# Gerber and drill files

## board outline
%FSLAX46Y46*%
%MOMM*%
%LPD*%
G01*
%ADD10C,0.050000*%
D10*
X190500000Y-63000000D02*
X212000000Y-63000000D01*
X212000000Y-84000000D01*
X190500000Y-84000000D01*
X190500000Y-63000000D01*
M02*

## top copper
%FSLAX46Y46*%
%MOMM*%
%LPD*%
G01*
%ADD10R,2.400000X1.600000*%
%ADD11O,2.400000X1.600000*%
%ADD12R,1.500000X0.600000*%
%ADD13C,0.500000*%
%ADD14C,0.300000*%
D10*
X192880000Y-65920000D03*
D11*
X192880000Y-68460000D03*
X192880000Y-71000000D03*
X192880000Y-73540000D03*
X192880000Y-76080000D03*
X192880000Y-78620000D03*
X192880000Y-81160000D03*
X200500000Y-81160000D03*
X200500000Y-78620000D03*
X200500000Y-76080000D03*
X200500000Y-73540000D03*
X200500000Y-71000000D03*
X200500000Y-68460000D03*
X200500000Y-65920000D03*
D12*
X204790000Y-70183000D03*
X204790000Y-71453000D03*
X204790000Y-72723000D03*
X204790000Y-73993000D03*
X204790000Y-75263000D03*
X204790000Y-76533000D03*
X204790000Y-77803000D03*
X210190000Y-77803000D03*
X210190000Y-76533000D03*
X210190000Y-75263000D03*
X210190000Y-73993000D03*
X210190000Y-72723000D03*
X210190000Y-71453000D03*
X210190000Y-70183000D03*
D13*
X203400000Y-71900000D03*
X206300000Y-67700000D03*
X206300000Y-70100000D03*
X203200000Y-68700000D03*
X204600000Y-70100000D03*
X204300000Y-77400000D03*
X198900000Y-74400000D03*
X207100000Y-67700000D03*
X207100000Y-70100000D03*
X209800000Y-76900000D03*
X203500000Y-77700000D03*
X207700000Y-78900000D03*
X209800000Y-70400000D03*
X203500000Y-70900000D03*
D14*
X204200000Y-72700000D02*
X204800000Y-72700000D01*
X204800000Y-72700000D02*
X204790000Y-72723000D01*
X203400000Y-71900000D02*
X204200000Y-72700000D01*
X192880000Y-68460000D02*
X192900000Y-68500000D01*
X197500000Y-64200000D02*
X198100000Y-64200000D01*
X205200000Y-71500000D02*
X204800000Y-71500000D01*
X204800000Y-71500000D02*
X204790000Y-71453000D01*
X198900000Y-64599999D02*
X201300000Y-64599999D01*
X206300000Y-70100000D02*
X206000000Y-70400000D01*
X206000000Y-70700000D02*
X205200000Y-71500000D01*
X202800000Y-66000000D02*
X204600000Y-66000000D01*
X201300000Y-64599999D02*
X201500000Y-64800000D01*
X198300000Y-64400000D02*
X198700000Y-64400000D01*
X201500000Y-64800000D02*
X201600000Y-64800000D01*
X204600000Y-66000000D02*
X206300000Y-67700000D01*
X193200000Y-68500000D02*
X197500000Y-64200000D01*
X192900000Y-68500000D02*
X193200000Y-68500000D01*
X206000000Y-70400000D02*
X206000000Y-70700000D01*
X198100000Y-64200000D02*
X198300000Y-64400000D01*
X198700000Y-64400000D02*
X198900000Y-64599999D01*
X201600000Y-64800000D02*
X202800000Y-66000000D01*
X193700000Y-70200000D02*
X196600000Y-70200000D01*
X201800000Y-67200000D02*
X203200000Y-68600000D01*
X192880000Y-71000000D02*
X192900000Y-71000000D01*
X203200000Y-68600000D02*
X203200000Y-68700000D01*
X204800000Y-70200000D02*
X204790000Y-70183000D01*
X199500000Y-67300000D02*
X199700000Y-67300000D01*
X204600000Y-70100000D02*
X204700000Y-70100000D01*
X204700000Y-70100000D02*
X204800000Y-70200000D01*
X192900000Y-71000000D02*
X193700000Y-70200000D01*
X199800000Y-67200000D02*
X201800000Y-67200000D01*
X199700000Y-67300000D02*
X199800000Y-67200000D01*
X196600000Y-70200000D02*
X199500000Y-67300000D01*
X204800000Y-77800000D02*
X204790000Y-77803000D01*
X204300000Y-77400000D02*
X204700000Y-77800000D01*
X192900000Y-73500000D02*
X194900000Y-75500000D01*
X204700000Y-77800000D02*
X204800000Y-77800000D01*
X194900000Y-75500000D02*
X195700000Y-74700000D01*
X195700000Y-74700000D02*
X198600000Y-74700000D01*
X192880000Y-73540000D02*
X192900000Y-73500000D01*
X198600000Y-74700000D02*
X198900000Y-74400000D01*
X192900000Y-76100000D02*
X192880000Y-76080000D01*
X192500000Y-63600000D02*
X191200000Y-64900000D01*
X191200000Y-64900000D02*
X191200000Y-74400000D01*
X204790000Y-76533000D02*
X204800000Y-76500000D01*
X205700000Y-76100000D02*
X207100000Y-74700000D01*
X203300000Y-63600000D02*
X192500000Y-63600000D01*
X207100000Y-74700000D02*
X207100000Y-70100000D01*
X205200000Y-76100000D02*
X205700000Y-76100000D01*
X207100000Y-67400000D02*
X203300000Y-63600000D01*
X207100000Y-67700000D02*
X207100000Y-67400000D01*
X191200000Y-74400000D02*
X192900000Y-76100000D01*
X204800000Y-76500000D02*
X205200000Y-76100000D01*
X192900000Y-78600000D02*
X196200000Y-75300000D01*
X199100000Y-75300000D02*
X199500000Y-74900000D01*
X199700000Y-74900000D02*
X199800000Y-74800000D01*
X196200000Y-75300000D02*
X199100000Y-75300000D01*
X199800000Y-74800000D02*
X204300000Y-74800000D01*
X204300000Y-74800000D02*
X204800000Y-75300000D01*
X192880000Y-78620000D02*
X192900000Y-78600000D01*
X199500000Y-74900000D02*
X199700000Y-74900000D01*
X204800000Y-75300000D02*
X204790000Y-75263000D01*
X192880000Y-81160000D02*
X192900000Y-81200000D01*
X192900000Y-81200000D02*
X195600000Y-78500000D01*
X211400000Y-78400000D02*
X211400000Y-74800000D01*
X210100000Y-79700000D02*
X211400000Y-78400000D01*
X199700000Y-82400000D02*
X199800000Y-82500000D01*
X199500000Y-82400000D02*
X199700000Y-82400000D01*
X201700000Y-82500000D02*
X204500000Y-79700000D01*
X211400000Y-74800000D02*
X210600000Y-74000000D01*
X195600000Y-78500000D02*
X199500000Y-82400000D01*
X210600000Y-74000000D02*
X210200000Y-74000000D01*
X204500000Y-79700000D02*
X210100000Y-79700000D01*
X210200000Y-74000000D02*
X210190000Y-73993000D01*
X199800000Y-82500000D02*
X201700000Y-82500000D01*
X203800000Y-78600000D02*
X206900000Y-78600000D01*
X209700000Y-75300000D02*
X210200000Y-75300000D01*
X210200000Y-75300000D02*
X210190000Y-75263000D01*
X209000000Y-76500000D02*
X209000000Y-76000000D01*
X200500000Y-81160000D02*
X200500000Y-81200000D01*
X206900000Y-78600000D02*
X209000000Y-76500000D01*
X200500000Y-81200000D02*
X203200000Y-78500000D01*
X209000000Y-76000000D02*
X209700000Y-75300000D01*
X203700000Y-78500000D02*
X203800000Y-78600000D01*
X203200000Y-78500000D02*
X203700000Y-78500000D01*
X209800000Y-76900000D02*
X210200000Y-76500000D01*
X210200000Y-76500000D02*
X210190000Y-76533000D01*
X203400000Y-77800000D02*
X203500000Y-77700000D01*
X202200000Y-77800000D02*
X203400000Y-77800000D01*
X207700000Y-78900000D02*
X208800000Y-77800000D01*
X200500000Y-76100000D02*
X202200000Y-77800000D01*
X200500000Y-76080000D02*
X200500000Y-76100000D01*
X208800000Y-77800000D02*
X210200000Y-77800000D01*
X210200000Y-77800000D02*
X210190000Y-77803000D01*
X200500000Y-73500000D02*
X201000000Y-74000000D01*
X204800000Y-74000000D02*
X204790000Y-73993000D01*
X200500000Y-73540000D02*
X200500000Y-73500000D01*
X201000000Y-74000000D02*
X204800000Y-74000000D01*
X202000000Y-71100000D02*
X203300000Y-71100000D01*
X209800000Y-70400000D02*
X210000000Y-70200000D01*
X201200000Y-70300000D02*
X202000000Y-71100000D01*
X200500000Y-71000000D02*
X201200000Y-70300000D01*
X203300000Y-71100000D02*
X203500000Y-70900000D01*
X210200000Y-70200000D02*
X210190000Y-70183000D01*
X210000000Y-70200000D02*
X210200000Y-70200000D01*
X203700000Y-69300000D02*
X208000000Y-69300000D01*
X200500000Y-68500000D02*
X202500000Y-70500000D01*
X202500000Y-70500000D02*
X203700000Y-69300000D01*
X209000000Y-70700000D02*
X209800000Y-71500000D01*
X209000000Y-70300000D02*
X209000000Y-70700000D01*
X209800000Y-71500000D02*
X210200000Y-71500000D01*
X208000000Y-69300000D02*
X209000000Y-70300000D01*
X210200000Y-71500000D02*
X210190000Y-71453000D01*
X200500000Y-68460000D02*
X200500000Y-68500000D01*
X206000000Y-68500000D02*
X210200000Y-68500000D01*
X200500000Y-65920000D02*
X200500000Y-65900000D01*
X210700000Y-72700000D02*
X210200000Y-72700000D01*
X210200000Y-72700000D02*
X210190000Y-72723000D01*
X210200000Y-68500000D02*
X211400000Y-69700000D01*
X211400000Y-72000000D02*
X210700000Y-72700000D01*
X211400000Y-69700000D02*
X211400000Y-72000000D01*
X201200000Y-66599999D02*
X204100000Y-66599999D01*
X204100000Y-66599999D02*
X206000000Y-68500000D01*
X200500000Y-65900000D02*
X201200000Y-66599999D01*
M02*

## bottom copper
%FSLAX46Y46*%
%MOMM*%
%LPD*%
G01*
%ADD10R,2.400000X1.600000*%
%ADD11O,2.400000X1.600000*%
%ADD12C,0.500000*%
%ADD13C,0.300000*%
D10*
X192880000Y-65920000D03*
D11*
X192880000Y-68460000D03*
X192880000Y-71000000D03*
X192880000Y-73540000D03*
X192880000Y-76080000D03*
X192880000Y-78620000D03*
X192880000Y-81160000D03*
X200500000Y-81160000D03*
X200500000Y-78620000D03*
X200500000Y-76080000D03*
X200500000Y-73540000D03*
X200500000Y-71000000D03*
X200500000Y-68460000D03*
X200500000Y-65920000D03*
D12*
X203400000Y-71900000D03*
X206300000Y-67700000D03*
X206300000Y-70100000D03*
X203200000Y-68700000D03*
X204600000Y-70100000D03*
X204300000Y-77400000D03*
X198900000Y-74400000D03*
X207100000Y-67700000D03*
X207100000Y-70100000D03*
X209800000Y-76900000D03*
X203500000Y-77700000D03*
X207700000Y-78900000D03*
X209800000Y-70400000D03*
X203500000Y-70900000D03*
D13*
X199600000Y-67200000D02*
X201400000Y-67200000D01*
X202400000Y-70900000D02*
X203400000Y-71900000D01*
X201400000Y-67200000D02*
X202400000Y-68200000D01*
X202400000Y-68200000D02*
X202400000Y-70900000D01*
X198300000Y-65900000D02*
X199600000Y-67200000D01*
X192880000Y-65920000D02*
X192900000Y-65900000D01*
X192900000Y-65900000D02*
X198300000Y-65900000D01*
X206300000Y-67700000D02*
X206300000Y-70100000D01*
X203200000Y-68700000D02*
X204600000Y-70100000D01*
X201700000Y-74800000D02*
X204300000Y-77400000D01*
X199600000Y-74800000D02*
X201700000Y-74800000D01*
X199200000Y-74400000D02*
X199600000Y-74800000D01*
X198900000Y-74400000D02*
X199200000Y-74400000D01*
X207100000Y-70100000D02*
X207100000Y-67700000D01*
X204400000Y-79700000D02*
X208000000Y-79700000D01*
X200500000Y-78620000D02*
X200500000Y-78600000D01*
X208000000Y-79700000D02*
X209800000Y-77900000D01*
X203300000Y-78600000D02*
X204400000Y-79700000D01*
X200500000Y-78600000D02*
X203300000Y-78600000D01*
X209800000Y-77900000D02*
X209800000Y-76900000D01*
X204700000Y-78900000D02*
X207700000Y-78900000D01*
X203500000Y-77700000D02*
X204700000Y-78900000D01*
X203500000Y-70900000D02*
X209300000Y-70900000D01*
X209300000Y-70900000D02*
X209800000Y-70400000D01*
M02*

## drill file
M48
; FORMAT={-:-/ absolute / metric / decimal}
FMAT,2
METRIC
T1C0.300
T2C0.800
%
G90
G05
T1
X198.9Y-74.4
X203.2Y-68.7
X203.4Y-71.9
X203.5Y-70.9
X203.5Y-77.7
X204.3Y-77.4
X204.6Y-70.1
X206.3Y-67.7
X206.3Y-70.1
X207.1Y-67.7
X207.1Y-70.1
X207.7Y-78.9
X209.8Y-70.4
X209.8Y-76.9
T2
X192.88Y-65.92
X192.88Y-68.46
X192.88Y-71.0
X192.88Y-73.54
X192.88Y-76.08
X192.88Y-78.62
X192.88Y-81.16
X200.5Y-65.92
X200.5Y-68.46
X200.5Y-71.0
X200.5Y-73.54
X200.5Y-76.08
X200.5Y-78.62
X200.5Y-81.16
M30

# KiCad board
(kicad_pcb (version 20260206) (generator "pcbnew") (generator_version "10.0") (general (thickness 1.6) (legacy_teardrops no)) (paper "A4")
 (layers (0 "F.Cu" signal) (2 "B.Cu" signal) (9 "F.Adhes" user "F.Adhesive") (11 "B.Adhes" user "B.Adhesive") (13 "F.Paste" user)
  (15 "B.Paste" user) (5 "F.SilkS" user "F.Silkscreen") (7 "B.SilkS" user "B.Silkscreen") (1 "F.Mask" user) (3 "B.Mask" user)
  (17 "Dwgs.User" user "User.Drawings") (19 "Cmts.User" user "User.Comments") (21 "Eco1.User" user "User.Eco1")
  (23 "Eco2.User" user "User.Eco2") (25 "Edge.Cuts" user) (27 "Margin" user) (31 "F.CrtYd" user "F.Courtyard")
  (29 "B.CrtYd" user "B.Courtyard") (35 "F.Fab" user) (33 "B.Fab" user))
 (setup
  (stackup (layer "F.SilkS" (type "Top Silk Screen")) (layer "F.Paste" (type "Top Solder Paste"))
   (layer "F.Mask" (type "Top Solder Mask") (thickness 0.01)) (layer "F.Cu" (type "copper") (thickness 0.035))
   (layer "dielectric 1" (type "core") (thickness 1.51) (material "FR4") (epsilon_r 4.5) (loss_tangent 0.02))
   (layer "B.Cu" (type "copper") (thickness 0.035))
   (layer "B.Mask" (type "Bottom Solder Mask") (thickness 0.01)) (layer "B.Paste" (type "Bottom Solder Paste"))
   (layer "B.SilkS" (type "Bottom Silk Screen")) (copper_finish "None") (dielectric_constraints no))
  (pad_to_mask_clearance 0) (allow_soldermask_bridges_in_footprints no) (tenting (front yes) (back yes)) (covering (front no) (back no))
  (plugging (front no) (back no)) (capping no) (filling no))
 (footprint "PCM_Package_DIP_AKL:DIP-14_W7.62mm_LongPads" (layer "F.Cu") (at 192.88 65.92)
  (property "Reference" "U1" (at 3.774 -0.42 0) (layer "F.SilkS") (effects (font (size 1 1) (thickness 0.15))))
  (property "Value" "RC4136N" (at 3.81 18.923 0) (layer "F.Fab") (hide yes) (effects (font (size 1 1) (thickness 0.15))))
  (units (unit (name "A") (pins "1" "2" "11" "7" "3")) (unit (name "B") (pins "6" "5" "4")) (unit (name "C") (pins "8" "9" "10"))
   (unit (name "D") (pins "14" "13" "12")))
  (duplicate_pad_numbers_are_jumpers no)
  (pad "1" thru_hole rect (at 0 0) (size 2.4 1.6) (drill 0.8) (layers "*.Cu" "*.Mask") (remove_unused_layers no) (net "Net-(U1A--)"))
  (pad "2" thru_hole oval (at 0 2.54) (size 2.4 1.6) (drill 0.8) (layers "*.Cu" "*.Mask") (remove_unused_layers no) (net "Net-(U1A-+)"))
  (pad "3" thru_hole oval (at 0 5.08) (size 2.4 1.6) (drill 0.8) (layers "*.Cu" "*.Mask") (remove_unused_layers no) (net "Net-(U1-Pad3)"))
  (pad "4" thru_hole oval (at 0 7.62) (size 2.4 1.6) (drill 0.8) (layers "*.Cu" "*.Mask") (remove_unused_layers no) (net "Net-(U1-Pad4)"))
  (pad "5" thru_hole oval (at 0 10.16) (size 2.4 1.6) (drill 0.8) (layers "*.Cu" "*.Mask") (remove_unused_layers no) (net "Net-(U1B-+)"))
  (pad "6" thru_hole oval (at 0 12.7) (size 2.4 1.6) (drill 0.8) (layers "*.Cu" "*.Mask") (remove_unused_layers no) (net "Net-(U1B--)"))
  (pad "7" thru_hole oval (at 0 15.24) (size 2.4 1.6) (drill 0.8) (layers "*.Cu" "*.Mask") (remove_unused_layers no) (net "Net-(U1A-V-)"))
  (pad "8" thru_hole oval (at 7.62 15.24) (size 2.4 1.6) (drill 0.8) (layers "*.Cu" "*.Mask") (remove_unused_layers no) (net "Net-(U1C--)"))
  (pad "9" thru_hole oval (at 7.62 12.7) (size 2.4 1.6) (drill 0.8) (layers "*.Cu" "*.Mask") (remove_unused_layers no) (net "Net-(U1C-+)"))
  (pad "10" thru_hole oval (at 7.62 10.16) (size 2.4 1.6) (drill 0.8) (layers "*.Cu" "*.Mask") (remove_unused_layers no)
   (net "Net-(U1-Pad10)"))
  (pad "11" thru_hole oval (at 7.62 7.62) (size 2.4 1.6) (drill 0.8) (layers "*.Cu" "*.Mask") (remove_unused_layers no) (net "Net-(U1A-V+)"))
  (pad "12" thru_hole oval (at 7.62 5.08) (size 2.4 1.6) (drill 0.8) (layers "*.Cu" "*.Mask") (remove_unused_layers no)
   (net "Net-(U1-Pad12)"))
  (pad "13" thru_hole oval (at 7.62 2.54) (size 2.4 1.6) (drill 0.8) (layers "*.Cu" "*.Mask") (remove_unused_layers no) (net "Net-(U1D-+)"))
  (pad "14" thru_hole oval (at 7.62 0) (size 2.4 1.6) (drill 0.8) (layers "*.Cu" "*.Mask") (remove_unused_layers no) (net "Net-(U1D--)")))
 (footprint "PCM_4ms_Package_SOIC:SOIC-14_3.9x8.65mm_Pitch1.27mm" (layer "F.Cu") (at 207.5 74)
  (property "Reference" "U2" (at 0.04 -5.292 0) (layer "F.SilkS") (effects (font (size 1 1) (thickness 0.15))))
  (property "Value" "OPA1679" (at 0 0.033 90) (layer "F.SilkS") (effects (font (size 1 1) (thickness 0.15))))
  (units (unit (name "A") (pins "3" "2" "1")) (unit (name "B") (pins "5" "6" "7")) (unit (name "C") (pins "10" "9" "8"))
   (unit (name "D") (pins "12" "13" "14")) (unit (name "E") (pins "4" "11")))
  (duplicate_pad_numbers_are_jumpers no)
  (pad "1" smd rect (at -2.71 -3.817) (size 1.5 0.6) (layers "F.Cu" "F.Mask" "F.Paste") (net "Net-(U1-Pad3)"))
  (pad "2" smd rect (at -2.71 -2.547) (size 1.5 0.6) (layers "F.Cu" "F.Mask" "F.Paste") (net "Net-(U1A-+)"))
  (pad "3" smd rect (at -2.71 -1.277) (size 1.5 0.6) (layers "F.Cu" "F.Mask" "F.Paste") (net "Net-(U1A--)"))
  (pad "4" smd rect (at -2.71 -0.007) (size 1.5 0.6) (layers "F.Cu" "F.Mask" "F.Paste") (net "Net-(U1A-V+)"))
  (pad "5" smd rect (at -2.71 1.263) (size 1.5 0.6) (layers "F.Cu" "F.Mask" "F.Paste") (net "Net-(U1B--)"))
  (pad "6" smd rect (at -2.71 2.533) (size 1.5 0.6) (layers "F.Cu" "F.Mask" "F.Paste") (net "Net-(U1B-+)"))
  (pad "7" smd rect (at -2.71 3.803) (size 1.5 0.6) (layers "F.Cu" "F.Mask" "F.Paste") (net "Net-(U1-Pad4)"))
  (pad "8" smd rect (at 2.69 3.803) (size 1.5 0.6) (layers "F.Cu" "F.Mask" "F.Paste") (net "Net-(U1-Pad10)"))
  (pad "9" smd rect (at 2.69 2.533) (size 1.5 0.6) (layers "F.Cu" "F.Mask" "F.Paste") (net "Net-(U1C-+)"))
  (pad "10" smd rect (at 2.69 1.263) (size 1.5 0.6) (layers "F.Cu" "F.Mask" "F.Paste") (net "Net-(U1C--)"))
  (pad "11" smd rect (at 2.69 -0.007) (size 1.5 0.6) (layers "F.Cu" "F.Mask" "F.Paste") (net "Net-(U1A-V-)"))
  (pad "12" smd rect (at 2.69 -1.277) (size 1.5 0.6) (layers "F.Cu" "F.Mask" "F.Paste") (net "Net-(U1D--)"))
  (pad "13" smd rect (at 2.69 -2.547) (size 1.5 0.6) (layers "F.Cu" "F.Mask" "F.Paste") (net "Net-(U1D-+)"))
  (pad "14" smd rect (at 2.69 -3.817) (size 1.5 0.6) (layers "F.Cu" "F.Mask" "F.Paste") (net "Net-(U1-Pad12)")))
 (gr_rect (start 190.5 63) (end 212 84) (stroke (width 0.05) (type default)) (fill no) (layer "Edge.Cuts"))
 (segment (start 204.2 72.7) (end 204.8 72.7) (width 0.3) (layer "F.Cu") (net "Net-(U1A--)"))
 (segment (start 204.8 72.7) (end 204.79 72.723) (width 0.3) (layer "F.Cu") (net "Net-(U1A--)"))
 (segment (start 203.4 71.9) (end 204.2 72.7) (width 0.3) (layer "F.Cu") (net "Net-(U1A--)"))
 (via (at 203.4 71.9) (size 0.5) (drill 0.3) (layers "F.Cu" "B.Cu") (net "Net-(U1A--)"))
 (segment (start 199.6 67.2) (end 201.4 67.2) (width 0.3) (layer "B.Cu") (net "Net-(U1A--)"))
 (segment (start 202.4 70.9) (end 203.4 71.9) (width 0.3) (layer "B.Cu") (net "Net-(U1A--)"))
 (segment (start 201.4 67.2) (end 202.4 68.2) (width 0.3) (layer "B.Cu") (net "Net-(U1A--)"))
 (segment (start 202.4 68.2) (end 202.4 70.9) (width 0.3) (layer "B.Cu") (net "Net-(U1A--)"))
 (segment (start 198.3 65.9) (end 199.6 67.2) (width 0.3) (layer "B.Cu") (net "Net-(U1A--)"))
 (segment (start 192.88 65.92) (end 192.9 65.9) (width 0.3) (layer "B.Cu") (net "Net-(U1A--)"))
 (segment (start 192.9 65.9) (end 198.3 65.9) (width 0.3) (layer "B.Cu") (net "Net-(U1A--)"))
 (segment (start 192.88 68.46) (end 192.9 68.5) (width 0.3) (layer "F.Cu") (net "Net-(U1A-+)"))
 (segment (start 197.5 64.2) (end 198.1 64.2) (width 0.3) (layer "F.Cu") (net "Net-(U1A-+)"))
 (segment (start 205.2 71.5) (end 204.8 71.5) (width 0.3) (layer "F.Cu") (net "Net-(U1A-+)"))
 (segment (start 204.8 71.5) (end 204.79 71.453) (width 0.3) (layer "F.Cu") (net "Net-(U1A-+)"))
 (segment (start 198.9 64.599999) (end 201.3 64.599999) (width 0.3) (layer "F.Cu") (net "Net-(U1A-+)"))
 (segment (start 206.3 70.1) (end 206 70.4) (width 0.3) (layer "F.Cu") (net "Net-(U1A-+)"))
 (segment (start 206 70.7) (end 205.2 71.5) (width 0.3) (layer "F.Cu") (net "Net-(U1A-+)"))
 (segment (start 202.8 66) (end 204.6 66) (width 0.3) (layer "F.Cu") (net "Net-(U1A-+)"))
 (segment (start 201.3 64.599999) (end 201.5 64.8) (width 0.3) (layer "F.Cu") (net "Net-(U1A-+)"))
 (segment (start 198.3 64.4) (end 198.7 64.4) (width 0.3) (layer "F.Cu") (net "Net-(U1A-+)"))
 (segment (start 201.5 64.8) (end 201.6 64.8) (width 0.3) (layer "F.Cu") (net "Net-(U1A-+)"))
 (segment (start 204.6 66) (end 206.3 67.7) (width 0.3) (layer "F.Cu") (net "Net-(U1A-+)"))
 (segment (start 193.2 68.5) (end 197.5 64.2) (width 0.3) (layer "F.Cu") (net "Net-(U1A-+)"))
 (segment (start 192.9 68.5) (end 193.2 68.5) (width 0.3) (layer "F.Cu") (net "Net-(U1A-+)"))
 (segment (start 206 70.4) (end 206 70.7) (width 0.3) (layer "F.Cu") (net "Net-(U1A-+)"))
 (segment (start 198.1 64.2) (end 198.3 64.4) (width 0.3) (layer "F.Cu") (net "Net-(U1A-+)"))
 (segment (start 198.7 64.4) (end 198.9 64.599999) (width 0.3) (layer "F.Cu") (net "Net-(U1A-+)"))
 (segment (start 201.6 64.8) (end 202.8 66) (width 0.3) (layer "F.Cu") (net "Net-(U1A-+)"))
 (via (at 206.3 67.7) (size 0.5) (drill 0.3) (layers "F.Cu" "B.Cu") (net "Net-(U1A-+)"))
 (via (at 206.3 70.1) (size 0.5) (drill 0.3) (layers "F.Cu" "B.Cu") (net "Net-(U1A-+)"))
 (segment (start 206.3 67.7) (end 206.3 70.1) (width 0.3) (layer "B.Cu") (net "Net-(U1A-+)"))
 (segment (start 193.7 70.2) (end 196.6 70.2) (width 0.3) (layer "F.Cu") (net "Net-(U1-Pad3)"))
 (segment (start 201.8 67.2) (end 203.2 68.6) (width 0.3) (layer "F.Cu") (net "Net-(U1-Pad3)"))
 (segment (start 192.88 71) (end 192.9 71) (width 0.3) (layer "F.Cu") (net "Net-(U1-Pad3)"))
 (segment (start 203.2 68.6) (end 203.2 68.7) (width 0.3) (layer "F.Cu") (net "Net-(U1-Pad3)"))
 (segment (start 204.8 70.2) (end 204.79 70.183) (width 0.3) (layer "F.Cu") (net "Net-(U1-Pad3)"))
 (segment (start 199.5 67.3) (end 199.7 67.3) (width 0.3) (layer "F.Cu") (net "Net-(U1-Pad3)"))
 (segment (start 204.6 70.1) (end 204.7 70.1) (width 0.3) (layer "F.Cu") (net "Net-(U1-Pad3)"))
 (segment (start 204.7 70.1) (end 204.8 70.2) (width 0.3) (layer "F.Cu") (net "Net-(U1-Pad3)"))
 (segment (start 192.9 71) (end 193.7 70.2) (width 0.3) (layer "F.Cu") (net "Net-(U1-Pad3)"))
 (segment (start 199.8 67.2) (end 201.8 67.2) (width 0.3) (layer "F.Cu") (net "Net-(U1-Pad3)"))
 (segment (start 199.7 67.3) (end 199.8 67.2) (width 0.3) (layer "F.Cu") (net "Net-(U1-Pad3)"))
 (segment (start 196.6 70.2) (end 199.5 67.3) (width 0.3) (layer "F.Cu") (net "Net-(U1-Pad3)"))
 (via (at 203.2 68.7) (size 0.5) (drill 0.3) (layers "F.Cu" "B.Cu") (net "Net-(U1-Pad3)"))
 (via (at 204.6 70.1) (size 0.5) (drill 0.3) (layers "F.Cu" "B.Cu") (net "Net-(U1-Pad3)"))
 (segment (start 203.2 68.7) (end 204.6 70.1) (width 0.3) (layer "B.Cu") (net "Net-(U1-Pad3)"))
 (segment (start 204.8 77.8) (end 204.79 77.803) (width 0.3) (layer "F.Cu") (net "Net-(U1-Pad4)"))
 (segment (start 204.3 77.4) (end 204.7 77.8) (width 0.3) (layer "F.Cu") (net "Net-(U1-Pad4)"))
 (segment (start 192.9 73.5) (end 194.9 75.5) (width 0.3) (layer "F.Cu") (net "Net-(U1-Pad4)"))
 (segment (start 204.7 77.8) (end 204.8 77.8) (width 0.3) (layer "F.Cu") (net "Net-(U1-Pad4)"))
 (segment (start 194.9 75.5) (end 195.7 74.7) (width 0.3) (layer "F.Cu") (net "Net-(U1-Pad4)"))
 (segment (start 195.7 74.7) (end 198.6 74.7) (width 0.3) (layer "F.Cu") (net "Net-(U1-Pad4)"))
 (segment (start 192.88 73.54) (end 192.9 73.5) (width 0.3) (layer "F.Cu") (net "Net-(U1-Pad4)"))
 (segment (start 198.6 74.7) (end 198.9 74.4) (width 0.3) (layer "F.Cu") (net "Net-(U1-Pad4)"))
 (via (at 204.3 77.4) (size 0.5) (drill 0.3) (layers "F.Cu" "B.Cu") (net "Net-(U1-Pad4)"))
 (via (at 198.9 74.4) (size 0.5) (drill 0.3) (layers "F.Cu" "B.Cu") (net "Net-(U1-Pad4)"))
 (segment (start 201.7 74.8) (end 204.3 77.4) (width 0.3) (layer "B.Cu") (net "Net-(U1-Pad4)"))
 (segment (start 199.6 74.8) (end 201.7 74.8) (width 0.3) (layer "B.Cu") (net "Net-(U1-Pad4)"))
 (segment (start 199.2 74.4) (end 199.6 74.8) (width 0.3) (layer "B.Cu") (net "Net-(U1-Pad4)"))
 (segment (start 198.9 74.4) (end 199.2 74.4) (width 0.3) (layer "B.Cu") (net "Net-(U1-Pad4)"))
 (segment (start 192.9 76.1) (end 192.88 76.08) (width 0.3) (layer "F.Cu") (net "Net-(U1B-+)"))
 (segment (start 192.5 63.6) (end 191.2 64.9) (width 0.3) (layer "F.Cu") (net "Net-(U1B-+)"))
 (segment (start 191.2 64.9) (end 191.2 74.4) (width 0.3) (layer "F.Cu") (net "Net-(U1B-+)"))
 (segment (start 204.79 76.533) (end 204.8 76.5) (width 0.3) (layer "F.Cu") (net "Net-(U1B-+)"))
 (segment (start 205.7 76.1) (end 207.1 74.7) (width 0.3) (layer "F.Cu") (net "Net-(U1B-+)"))
 (segment (start 203.3 63.6) (end 192.5 63.6) (width 0.3) (layer "F.Cu") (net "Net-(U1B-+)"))
 (segment (start 207.1 74.7) (end 207.1 70.1) (width 0.3) (layer "F.Cu") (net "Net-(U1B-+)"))
 (segment (start 205.2 76.1) (end 205.7 76.1) (width 0.3) (layer "F.Cu") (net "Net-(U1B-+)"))
 (segment (start 207.1 67.4) (end 203.3 63.6) (width 0.3) (layer "F.Cu") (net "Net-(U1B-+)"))
 (segment (start 207.1 67.7) (end 207.1 67.4) (width 0.3) (layer "F.Cu") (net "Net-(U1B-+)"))
 (segment (start 191.2 74.4) (end 192.9 76.1) (width 0.3) (layer "F.Cu") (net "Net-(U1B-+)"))
 (segment (start 204.8 76.5) (end 205.2 76.1) (width 0.3) (layer "F.Cu") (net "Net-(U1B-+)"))
 (via (at 207.1 67.7) (size 0.5) (drill 0.3) (layers "F.Cu" "B.Cu") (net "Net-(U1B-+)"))
 (via (at 207.1 70.1) (size 0.5) (drill 0.3) (layers "F.Cu" "B.Cu") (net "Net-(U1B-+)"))
 (segment (start 207.1 70.1) (end 207.1 67.7) (width 0.3) (layer "B.Cu") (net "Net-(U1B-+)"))
 (segment (start 192.9 78.6) (end 196.2 75.3) (width 0.3) (layer "F.Cu") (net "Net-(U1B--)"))
 (segment (start 199.1 75.3) (end 199.5 74.9) (width 0.3) (layer "F.Cu") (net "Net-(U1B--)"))
 (segment (start 199.7 74.9) (end 199.8 74.8) (width 0.3) (layer "F.Cu") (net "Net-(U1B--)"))
 (segment (start 196.2 75.3) (end 199.1 75.3) (width 0.3) (layer "F.Cu") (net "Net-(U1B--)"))
 (segment (start 199.8 74.8) (end 204.3 74.8) (width 0.3) (layer "F.Cu") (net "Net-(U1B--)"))
 (segment (start 204.3 74.8) (end 204.8 75.3) (width 0.3) (layer "F.Cu") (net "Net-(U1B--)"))
 (segment (start 192.88 78.62) (end 192.9 78.6) (width 0.3) (layer "F.Cu") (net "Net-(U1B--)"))
 (segment (start 199.5 74.9) (end 199.7 74.9) (width 0.3) (layer "F.Cu") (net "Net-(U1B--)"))
 (segment (start 204.8 75.3) (end 204.79 75.263) (width 0.3) (layer "F.Cu") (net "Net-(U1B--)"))
 (segment (start 192.88 81.16) (end 192.9 81.2) (width 0.3) (layer "F.Cu") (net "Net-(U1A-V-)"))
 (segment (start 192.9 81.2) (end 195.6 78.5) (width 0.3) (layer "F.Cu") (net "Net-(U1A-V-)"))
 (segment (start 211.4 78.4) (end 211.4 74.8) (width 0.3) (layer "F.Cu") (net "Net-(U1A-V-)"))
 (segment (start 210.1 79.7) (end 211.4 78.4) (width 0.3) (layer "F.Cu") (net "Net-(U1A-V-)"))
 (segment (start 199.7 82.4) (end 199.8 82.5) (width 0.3) (layer "F.Cu") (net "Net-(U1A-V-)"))
 (segment (start 199.5 82.4) (end 199.7 82.4) (width 0.3) (layer "F.Cu") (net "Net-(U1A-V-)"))
 (segment (start 201.7 82.5) (end 204.5 79.7) (width 0.3) (layer "F.Cu") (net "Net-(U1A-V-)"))
 (segment (start 211.4 74.8) (end 210.6 74) (width 0.3) (layer "F.Cu") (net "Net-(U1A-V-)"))
 (segment (start 195.6 78.5) (end 199.5 82.4) (width 0.3) (layer "F.Cu") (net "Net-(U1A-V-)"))
 (segment (start 210.6 74) (end 210.2 74) (width 0.3) (layer "F.Cu") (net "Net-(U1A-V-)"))
 (segment (start 204.5 79.7) (end 210.1 79.7) (width 0.3) (layer "F.Cu") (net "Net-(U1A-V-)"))
 (segment (start 210.2 74) (end 210.19 73.993) (width 0.3) (layer "F.Cu") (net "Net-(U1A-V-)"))
 (segment (start 199.8 82.5) (end 201.7 82.5) (width 0.3) (layer "F.Cu") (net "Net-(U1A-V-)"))
 (segment (start 203.8 78.6) (end 206.9 78.6) (width 0.3) (layer "F.Cu") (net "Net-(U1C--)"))
 (segment (start 209.7 75.3) (end 210.2 75.3) (width 0.3) (layer "F.Cu") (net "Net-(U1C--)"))
 (segment (start 210.2 75.3) (end 210.19 75.263) (width 0.3) (layer "F.Cu") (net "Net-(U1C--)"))
 (segment (start 209 76.5) (end 209 76) (width 0.3) (layer "F.Cu") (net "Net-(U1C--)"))
 (segment (start 200.5 81.16) (end 200.5 81.2) (width 0.3) (layer "F.Cu") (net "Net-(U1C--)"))
 (segment (start 206.9 78.6) (end 209 76.5) (width 0.3) (layer "F.Cu") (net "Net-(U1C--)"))
 (segment (start 200.5 81.2) (end 203.2 78.5) (width 0.3) (layer "F.Cu") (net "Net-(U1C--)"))
 (segment (start 209 76) (end 209.7 75.3) (width 0.3) (layer "F.Cu") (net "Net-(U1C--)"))
 (segment (start 203.7 78.5) (end 203.8 78.6) (width 0.3) (layer "F.Cu") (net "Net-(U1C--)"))
 (segment (start 203.2 78.5) (end 203.7 78.5) (width 0.3) (layer "F.Cu") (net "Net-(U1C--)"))
 (segment (start 209.8 76.9) (end 210.2 76.5) (width 0.3) (layer "F.Cu") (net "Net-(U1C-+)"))
 (segment (start 210.2 76.5) (end 210.19 76.533) (width 0.3) (layer "F.Cu") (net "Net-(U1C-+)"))
 (via (at 209.8 76.9) (size 0.5) (drill 0.3) (layers "F.Cu" "B.Cu") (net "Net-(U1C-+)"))
 (segment (start 204.4 79.7) (end 208 79.7) (width 0.3) (layer "B.Cu") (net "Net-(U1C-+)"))
 (segment (start 200.5 78.62) (end 200.5 78.6) (width 0.3) (layer "B.Cu") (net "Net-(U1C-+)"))
 (segment (start 208 79.7) (end 209.8 77.9) (width 0.3) (layer "B.Cu") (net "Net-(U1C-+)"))
 (segment (start 203.3 78.6) (end 204.4 79.7) (width 0.3) (layer "B.Cu") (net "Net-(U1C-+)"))
 (segment (start 200.5 78.6) (end 203.3 78.6) (width 0.3) (layer "B.Cu") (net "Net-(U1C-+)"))
 (segment (start 209.8 77.9) (end 209.8 76.9) (width 0.3) (layer "B.Cu") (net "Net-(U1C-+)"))
 (segment (start 203.4 77.8) (end 203.5 77.7) (width 0.3) (layer "F.Cu") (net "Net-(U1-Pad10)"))
 (segment (start 202.2 77.8) (end 203.4 77.8) (width 0.3) (layer "F.Cu") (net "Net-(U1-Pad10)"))
 (segment (start 207.7 78.9) (end 208.8 77.8) (width 0.3) (layer "F.Cu") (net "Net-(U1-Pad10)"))
 (segment (start 200.5 76.1) (end 202.2 77.8) (width 0.3) (layer "F.Cu") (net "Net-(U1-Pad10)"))
 (segment (start 200.5 76.08) (end 200.5 76.1) (width 0.3) (layer "F.Cu") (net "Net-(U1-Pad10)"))
 (segment (start 208.8 77.8) (end 210.2 77.8) (width 0.3) (layer "F.Cu") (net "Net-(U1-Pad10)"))
 (segment (start 210.2 77.8) (end 210.19 77.803) (width 0.3) (layer "F.Cu") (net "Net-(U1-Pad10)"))
 (via (at 203.5 77.7) (size 0.5) (drill 0.3) (layers "F.Cu" "B.Cu") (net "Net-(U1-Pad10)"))
 (via (at 207.7 78.9) (size 0.5) (drill 0.3) (layers "F.Cu" "B.Cu") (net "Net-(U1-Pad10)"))
 (segment (start 204.7 78.9) (end 207.7 78.9) (width 0.3) (layer "B.Cu") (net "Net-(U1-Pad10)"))
 (segment (start 203.5 77.7) (end 204.7 78.9) (width 0.3) (layer "B.Cu") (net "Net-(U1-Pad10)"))
 (segment (start 200.5 73.5) (end 201 74) (width 0.3) (layer "F.Cu") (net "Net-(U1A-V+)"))
 (segment (start 204.8 74) (end 204.79 73.993) (width 0.3) (layer "F.Cu") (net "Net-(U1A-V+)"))
 (segment (start 200.5 73.54) (end 200.5 73.5) (width 0.3) (layer "F.Cu") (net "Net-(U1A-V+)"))
 (segment (start 201 74) (end 204.8 74) (width 0.3) (layer "F.Cu") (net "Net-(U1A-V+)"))
 (segment (start 202 71.1) (end 203.3 71.1) (width 0.3) (layer "F.Cu") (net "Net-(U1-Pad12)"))
 (segment (start 209.8 70.4) (end 210 70.2) (width 0.3) (layer "F.Cu") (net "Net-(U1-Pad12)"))
 (segment (start 201.2 70.3) (end 202 71.1) (width 0.3) (layer "F.Cu") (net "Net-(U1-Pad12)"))
 (segment (start 200.5 71) (end 201.2 70.3) (width 0.3) (layer "F.Cu") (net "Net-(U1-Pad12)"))
 (segment (start 203.3 71.1) (end 203.5 70.9) (width 0.3) (layer "F.Cu") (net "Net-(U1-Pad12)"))
 (segment (start 210.2 70.2) (end 210.19 70.183) (width 0.3) (layer "F.Cu") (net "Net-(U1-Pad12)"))
 (segment (start 210 70.2) (end 210.2 70.2) (width 0.3) (layer "F.Cu") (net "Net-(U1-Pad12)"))
 (via (at 209.8 70.4) (size 0.5) (drill 0.3) (layers "F.Cu" "B.Cu") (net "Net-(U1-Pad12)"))
 (via (at 203.5 70.9) (size 0.5) (drill 0.3) (layers "F.Cu" "B.Cu") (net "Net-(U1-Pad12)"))
 (segment (start 203.5 70.9) (end 209.3 70.9) (width 0.3) (layer "B.Cu") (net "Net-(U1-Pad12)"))
 (segment (start 209.3 70.9) (end 209.8 70.4) (width 0.3) (layer "B.Cu") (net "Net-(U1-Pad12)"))
 (segment (start 203.7 69.3) (end 208 69.3) (width 0.3) (layer "F.Cu") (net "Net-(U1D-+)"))
 (segment (start 200.5 68.5) (end 202.5 70.5) (width 0.3) (layer "F.Cu") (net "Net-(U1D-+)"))
 (segment (start 202.5 70.5) (end 203.7 69.3) (width 0.3) (layer "F.Cu") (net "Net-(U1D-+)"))
 (segment (start 209 70.7) (end 209.8 71.5) (width 0.3) (layer "F.Cu") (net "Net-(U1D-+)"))
 (segment (start 209 70.3) (end 209 70.7) (width 0.3) (layer "F.Cu") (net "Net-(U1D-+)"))
 (segment (start 209.8 71.5) (end 210.2 71.5) (width 0.3) (layer "F.Cu") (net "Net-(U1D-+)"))
 (segment (start 208 69.3) (end 209 70.3) (width 0.3) (layer "F.Cu") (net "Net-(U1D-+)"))
 (segment (start 210.2 71.5) (end 210.19 71.453) (width 0.3) (layer "F.Cu") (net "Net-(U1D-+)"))
 (segment (start 200.5 68.46) (end 200.5 68.5) (width 0.3) (layer "F.Cu") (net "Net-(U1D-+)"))
 (segment (start 206 68.5) (end 210.2 68.5) (width 0.3) (layer "F.Cu") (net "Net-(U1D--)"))
 (segment (start 200.5 65.92) (end 200.5 65.9) (width 0.3) (layer "F.Cu") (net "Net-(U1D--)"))
 (segment (start 210.7 72.7) (end 210.2 72.7) (width 0.3) (layer "F.Cu") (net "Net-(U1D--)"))
 (segment (start 210.2 72.7) (end 210.19 72.723) (width 0.3) (layer "F.Cu") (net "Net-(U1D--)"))
 (segment (start 210.2 68.5) (end 211.4 69.7) (width 0.3) (layer "F.Cu") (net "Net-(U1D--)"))
 (segment (start 211.4 72) (end 210.7 72.7) (width 0.3) (layer "F.Cu") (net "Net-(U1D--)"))
 (segment (start 211.4 69.7) (end 211.4 72) (width 0.3) (layer "F.Cu") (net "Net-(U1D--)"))
 (segment (start 201.2 66.599999) (end 204.1 66.599999) (width 0.3) (layer "F.Cu") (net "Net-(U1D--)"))
 (segment (start 204.1 66.599999) (end 206 68.5) (width 0.3) (layer "F.Cu") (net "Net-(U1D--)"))
 (segment (start 200.5 65.9) (end 201.2 66.599999) (width 0.3) (layer "F.Cu") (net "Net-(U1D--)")))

